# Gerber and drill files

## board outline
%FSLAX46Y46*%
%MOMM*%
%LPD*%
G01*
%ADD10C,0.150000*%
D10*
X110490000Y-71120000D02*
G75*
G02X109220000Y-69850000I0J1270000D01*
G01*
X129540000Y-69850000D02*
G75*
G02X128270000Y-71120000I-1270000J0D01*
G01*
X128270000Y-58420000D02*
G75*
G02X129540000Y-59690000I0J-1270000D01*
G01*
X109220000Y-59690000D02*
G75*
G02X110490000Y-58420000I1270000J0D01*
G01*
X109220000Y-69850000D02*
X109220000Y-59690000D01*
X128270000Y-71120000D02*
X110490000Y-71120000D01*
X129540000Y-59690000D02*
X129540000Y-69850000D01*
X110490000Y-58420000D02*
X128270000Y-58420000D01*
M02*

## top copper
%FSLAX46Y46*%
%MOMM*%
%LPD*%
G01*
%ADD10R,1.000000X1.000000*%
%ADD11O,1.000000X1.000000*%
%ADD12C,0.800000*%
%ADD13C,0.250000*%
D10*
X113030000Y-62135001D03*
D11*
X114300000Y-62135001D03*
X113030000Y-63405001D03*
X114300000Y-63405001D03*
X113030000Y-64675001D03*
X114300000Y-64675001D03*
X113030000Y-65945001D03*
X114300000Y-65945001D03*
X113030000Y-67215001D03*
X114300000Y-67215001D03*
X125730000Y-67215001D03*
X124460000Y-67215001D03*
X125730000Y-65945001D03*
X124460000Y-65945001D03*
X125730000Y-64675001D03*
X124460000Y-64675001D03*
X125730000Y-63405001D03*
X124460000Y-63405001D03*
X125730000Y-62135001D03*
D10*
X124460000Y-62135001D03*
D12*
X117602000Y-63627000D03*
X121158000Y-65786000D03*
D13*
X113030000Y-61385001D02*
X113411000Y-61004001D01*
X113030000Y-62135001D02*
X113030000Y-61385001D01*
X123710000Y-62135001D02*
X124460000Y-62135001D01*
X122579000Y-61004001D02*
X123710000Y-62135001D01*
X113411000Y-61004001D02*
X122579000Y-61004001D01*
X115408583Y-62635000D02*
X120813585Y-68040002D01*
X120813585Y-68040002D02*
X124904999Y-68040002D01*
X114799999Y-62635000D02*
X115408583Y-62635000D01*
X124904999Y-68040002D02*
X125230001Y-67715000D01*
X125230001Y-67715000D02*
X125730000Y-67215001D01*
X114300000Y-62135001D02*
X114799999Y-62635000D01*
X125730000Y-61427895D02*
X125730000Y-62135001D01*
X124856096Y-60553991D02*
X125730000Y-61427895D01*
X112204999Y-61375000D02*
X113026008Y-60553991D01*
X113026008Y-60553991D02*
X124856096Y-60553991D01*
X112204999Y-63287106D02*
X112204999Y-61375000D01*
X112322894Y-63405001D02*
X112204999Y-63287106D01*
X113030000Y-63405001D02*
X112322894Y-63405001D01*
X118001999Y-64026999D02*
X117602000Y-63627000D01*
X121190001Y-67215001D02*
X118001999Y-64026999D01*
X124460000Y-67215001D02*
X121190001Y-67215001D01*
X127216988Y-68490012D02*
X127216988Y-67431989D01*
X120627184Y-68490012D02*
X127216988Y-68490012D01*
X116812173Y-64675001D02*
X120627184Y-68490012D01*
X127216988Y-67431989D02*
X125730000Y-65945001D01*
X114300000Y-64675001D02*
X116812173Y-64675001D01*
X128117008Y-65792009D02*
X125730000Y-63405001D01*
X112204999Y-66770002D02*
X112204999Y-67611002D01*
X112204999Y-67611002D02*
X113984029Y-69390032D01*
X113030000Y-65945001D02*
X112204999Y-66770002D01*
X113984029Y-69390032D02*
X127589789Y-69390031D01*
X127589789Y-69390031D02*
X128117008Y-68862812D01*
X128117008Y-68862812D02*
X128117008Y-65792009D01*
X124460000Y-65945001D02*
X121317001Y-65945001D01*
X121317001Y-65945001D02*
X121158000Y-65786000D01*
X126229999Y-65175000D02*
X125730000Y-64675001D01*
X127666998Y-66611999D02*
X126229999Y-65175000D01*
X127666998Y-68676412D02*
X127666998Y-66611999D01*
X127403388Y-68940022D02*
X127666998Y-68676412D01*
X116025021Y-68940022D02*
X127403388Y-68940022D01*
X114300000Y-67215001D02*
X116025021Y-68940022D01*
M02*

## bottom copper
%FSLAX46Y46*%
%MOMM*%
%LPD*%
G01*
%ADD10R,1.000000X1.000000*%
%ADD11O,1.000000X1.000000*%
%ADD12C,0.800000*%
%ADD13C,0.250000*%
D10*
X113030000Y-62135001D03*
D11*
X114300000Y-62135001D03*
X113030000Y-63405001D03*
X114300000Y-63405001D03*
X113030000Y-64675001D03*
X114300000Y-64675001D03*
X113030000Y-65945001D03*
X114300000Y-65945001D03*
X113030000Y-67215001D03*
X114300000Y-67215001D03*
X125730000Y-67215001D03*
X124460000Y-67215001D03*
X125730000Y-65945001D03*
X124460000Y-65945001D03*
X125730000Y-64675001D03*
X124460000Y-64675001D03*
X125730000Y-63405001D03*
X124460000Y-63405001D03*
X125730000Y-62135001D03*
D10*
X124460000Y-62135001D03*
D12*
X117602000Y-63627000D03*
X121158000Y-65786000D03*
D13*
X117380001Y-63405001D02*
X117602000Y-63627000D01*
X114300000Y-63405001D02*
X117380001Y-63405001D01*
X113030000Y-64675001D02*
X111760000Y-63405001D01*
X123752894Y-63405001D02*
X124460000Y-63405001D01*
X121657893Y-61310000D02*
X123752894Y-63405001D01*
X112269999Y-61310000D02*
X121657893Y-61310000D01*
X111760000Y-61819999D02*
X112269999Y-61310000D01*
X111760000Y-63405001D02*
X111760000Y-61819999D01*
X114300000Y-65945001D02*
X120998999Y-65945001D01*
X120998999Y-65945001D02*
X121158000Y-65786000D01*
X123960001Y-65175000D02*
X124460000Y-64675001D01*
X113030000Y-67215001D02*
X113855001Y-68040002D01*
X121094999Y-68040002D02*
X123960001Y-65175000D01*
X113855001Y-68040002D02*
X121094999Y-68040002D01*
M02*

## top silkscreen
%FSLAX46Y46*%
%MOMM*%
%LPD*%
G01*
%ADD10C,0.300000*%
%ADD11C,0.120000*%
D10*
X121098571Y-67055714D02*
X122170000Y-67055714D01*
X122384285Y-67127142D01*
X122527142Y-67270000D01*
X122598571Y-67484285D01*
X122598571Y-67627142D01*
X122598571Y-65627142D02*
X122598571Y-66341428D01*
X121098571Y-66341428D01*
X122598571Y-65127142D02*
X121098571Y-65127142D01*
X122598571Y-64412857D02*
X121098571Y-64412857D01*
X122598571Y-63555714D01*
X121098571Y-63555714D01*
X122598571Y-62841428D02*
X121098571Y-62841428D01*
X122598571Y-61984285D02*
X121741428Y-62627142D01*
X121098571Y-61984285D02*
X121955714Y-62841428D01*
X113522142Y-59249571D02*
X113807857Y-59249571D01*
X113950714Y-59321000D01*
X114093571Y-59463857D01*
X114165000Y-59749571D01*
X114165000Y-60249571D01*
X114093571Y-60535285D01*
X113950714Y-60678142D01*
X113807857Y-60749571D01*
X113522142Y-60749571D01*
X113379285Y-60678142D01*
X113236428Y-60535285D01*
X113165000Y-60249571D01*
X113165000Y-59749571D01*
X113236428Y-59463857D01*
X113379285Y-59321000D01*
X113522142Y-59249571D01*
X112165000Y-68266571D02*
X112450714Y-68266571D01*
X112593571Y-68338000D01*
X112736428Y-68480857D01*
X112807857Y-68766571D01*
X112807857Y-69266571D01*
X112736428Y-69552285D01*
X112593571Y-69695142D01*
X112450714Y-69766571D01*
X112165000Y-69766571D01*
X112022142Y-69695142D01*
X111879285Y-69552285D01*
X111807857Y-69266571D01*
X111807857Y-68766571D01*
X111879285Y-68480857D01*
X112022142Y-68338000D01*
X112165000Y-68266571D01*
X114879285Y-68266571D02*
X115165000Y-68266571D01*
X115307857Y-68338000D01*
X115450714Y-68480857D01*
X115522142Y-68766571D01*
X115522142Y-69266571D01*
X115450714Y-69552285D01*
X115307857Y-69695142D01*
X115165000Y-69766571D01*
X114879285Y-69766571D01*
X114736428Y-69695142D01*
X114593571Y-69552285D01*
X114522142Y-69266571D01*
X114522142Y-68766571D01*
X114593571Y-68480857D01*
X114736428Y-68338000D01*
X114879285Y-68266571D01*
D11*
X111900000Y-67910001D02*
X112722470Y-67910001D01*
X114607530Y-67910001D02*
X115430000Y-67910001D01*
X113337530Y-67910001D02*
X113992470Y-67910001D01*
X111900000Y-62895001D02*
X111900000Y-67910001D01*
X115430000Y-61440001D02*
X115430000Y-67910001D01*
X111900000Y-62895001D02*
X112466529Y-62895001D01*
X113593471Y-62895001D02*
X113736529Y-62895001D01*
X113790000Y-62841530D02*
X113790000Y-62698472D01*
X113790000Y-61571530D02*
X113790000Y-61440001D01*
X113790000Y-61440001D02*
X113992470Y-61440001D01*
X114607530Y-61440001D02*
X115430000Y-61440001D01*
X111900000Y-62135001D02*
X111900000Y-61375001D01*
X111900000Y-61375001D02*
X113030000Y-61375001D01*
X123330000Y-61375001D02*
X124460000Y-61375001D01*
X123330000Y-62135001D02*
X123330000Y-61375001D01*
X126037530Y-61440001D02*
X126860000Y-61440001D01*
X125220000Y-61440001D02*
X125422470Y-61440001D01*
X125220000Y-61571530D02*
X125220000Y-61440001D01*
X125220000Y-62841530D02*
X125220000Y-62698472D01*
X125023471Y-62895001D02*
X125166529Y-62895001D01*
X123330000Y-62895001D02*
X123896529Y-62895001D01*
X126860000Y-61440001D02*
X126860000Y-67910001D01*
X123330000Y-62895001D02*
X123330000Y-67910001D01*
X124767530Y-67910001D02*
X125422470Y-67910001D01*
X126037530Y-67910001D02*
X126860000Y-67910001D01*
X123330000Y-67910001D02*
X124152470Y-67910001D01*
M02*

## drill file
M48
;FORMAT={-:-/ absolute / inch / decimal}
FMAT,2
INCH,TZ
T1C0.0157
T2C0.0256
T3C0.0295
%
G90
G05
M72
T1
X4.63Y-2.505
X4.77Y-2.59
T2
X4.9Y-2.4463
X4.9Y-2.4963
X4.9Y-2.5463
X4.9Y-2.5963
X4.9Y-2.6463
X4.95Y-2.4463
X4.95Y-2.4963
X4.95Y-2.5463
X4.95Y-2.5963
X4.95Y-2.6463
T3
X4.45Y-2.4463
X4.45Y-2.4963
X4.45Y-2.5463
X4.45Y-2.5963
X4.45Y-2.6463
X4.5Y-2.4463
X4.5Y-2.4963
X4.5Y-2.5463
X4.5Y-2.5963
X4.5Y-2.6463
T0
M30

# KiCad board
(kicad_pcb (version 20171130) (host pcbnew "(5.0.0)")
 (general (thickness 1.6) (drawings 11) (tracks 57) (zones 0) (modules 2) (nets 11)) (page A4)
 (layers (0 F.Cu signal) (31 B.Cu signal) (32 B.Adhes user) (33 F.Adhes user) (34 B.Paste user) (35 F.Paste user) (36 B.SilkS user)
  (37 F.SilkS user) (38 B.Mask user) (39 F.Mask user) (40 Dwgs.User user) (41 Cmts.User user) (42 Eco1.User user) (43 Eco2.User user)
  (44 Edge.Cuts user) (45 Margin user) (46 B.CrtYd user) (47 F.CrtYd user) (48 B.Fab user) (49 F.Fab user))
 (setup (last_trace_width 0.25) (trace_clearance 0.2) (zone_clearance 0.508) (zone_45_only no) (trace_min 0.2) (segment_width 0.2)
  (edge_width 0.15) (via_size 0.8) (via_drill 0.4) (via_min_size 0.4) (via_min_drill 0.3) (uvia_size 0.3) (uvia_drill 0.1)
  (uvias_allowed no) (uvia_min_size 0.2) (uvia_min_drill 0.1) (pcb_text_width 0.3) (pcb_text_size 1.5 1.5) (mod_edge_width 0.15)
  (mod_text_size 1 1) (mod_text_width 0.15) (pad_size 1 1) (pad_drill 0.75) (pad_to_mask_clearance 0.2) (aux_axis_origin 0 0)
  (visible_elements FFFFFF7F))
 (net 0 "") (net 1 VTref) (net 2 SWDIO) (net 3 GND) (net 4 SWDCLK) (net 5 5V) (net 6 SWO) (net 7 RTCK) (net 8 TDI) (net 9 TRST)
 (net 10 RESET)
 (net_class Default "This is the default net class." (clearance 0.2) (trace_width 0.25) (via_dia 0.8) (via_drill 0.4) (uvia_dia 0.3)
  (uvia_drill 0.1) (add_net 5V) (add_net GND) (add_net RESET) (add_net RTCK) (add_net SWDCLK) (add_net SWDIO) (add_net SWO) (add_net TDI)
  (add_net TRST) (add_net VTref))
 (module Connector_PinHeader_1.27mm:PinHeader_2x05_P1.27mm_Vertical (layer F.Cu) (at 113.03 62.135001)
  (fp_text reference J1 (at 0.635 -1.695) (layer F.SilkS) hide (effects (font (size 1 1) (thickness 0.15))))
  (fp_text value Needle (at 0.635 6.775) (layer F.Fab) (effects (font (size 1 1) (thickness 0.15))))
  (fp_line (start -1.13 5.775) (end -0.30753 5.775) (layer F.SilkS) (width 0.12))
  (fp_line (start 1.57753 5.775) (end 2.4 5.775) (layer F.SilkS) (width 0.12))
  (fp_line (start 0.30753 5.775) (end 0.96247 5.775) (layer F.SilkS) (width 0.12))
  (fp_line (start -1.13 0.76) (end -1.13 5.775) (layer F.SilkS) (width 0.12))
  (fp_line (start 2.4 -0.695) (end 2.4 5.775) (layer F.SilkS) (width 0.12))
  (fp_line (start -1.13 0.76) (end -0.563471 0.76) (layer F.SilkS) (width 0.12))
  (fp_line (start 0.563471 0.76) (end 0.706529 0.76) (layer F.SilkS) (width 0.12))
  (fp_line (start 0.76 0.706529) (end 0.76 0.563471) (layer F.SilkS) (width 0.12))
  (fp_line (start 0.76 -0.563471) (end 0.76 -0.695) (layer F.SilkS) (width 0.12))
  (fp_line (start 0.76 -0.695) (end 0.96247 -0.695) (layer F.SilkS) (width 0.12))
  (fp_line (start 1.57753 -0.695) (end 2.4 -0.695) (layer F.SilkS) (width 0.12))
  (fp_line (start -1.13 0) (end -1.13 -0.76) (layer F.SilkS) (width 0.12))
  (fp_line (start -1.13 -0.76) (end 0 -0.76) (layer F.SilkS) (width 0.12))
  (pad 1 thru_hole rect (at 0 0) (size 1 1) (drill 0.75) (layers *.Cu *.Mask) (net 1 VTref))
  (pad 2 thru_hole oval (at 1.27 0) (size 1 1) (drill 0.75) (layers *.Cu *.Mask) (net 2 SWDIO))
  (pad 3 thru_hole oval (at 0 1.27) (size 1 1) (drill 0.75) (layers *.Cu *.Mask) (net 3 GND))
  (pad 4 thru_hole oval (at 1.27 1.27) (size 1 1) (drill 0.75) (layers *.Cu *.Mask) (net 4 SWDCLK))
  (pad 5 thru_hole oval (at 0 2.54) (size 1 1) (drill 0.75) (layers *.Cu *.Mask) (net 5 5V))
  (pad 6 thru_hole oval (at 1.27 2.54) (size 1 1) (drill 0.75) (layers *.Cu *.Mask) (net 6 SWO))
  (pad 7 thru_hole oval (at 0 3.81) (size 1 1) (drill 0.75) (layers *.Cu *.Mask) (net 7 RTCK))
  (pad 8 thru_hole oval (at 1.27 3.81) (size 1 1) (drill 0.75) (layers *.Cu *.Mask) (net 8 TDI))
  (pad 9 thru_hole oval (at 0 5.08) (size 1 1) (drill 0.75) (layers *.Cu *.Mask) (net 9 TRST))
  (pad 10 thru_hole oval (at 1.27 5.08) (size 1 1) (drill 0.75) (layers *.Cu *.Mask) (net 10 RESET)))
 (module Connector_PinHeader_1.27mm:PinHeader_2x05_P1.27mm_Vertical (layer F.Cu) (at 124.46 62.135001)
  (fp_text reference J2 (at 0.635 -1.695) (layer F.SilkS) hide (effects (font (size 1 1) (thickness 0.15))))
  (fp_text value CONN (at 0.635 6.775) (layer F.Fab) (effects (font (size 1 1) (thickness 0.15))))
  (fp_line (start -1.13 -0.76) (end 0 -0.76) (layer F.SilkS) (width 0.12))
  (fp_line (start -1.13 0) (end -1.13 -0.76) (layer F.SilkS) (width 0.12))
  (fp_line (start 1.57753 -0.695) (end 2.4 -0.695) (layer F.SilkS) (width 0.12))
  (fp_line (start 0.76 -0.695) (end 0.96247 -0.695) (layer F.SilkS) (width 0.12))
  (fp_line (start 0.76 -0.563471) (end 0.76 -0.695) (layer F.SilkS) (width 0.12))
  (fp_line (start 0.76 0.706529) (end 0.76 0.563471) (layer F.SilkS) (width 0.12))
  (fp_line (start 0.563471 0.76) (end 0.706529 0.76) (layer F.SilkS) (width 0.12))
  (fp_line (start -1.13 0.76) (end -0.563471 0.76) (layer F.SilkS) (width 0.12))
  (fp_line (start 2.4 -0.695) (end 2.4 5.775) (layer F.SilkS) (width 0.12))
  (fp_line (start -1.13 0.76) (end -1.13 5.775) (layer F.SilkS) (width 0.12))
  (fp_line (start 0.30753 5.775) (end 0.96247 5.775) (layer F.SilkS) (width 0.12))
  (fp_line (start 1.57753 5.775) (end 2.4 5.775) (layer F.SilkS) (width 0.12))
  (fp_line (start -1.13 5.775) (end -0.30753 5.775) (layer F.SilkS) (width 0.12))
  (pad 10 thru_hole oval (at 1.27 5.08) (size 1 1) (drill 0.65) (layers *.Cu *.Mask) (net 2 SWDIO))
  (pad 9 thru_hole oval (at 0 5.08) (size 1 1) (drill 0.65) (layers *.Cu *.Mask) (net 4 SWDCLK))
  (pad 8 thru_hole oval (at 1.27 3.81) (size 1 1) (drill 0.65) (layers *.Cu *.Mask) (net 6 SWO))
  (pad 7 thru_hole oval (at 0 3.81) (size 1 1) (drill 0.65) (layers *.Cu *.Mask) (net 8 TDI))
  (pad 6 thru_hole oval (at 1.27 2.54) (size 1 1) (drill 0.65) (layers *.Cu *.Mask) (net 10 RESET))
  (pad 5 thru_hole oval (at 0 2.54) (size 1 1) (drill 0.65) (layers *.Cu *.Mask) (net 9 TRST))
  (pad 4 thru_hole oval (at 1.27 1.27) (size 1 1) (drill 0.65) (layers *.Cu *.Mask) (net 7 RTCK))
  (pad 3 thru_hole oval (at 0 1.27) (size 1 1) (drill 0.65) (layers *.Cu *.Mask) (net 5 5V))
  (pad 2 thru_hole oval (at 1.27 0) (size 1 1) (drill 0.65) (layers *.Cu *.Mask) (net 3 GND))
  (pad 1 thru_hole rect (at 0 0) (size 1 1) (drill 0.65) (layers *.Cu *.Mask) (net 1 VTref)))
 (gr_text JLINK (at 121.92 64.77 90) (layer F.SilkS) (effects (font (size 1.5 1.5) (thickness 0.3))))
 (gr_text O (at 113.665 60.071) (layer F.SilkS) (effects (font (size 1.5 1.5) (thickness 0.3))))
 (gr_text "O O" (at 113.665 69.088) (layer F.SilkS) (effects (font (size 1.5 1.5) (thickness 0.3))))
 (gr_arc (start 110.49 69.85) (end 109.22 69.85) (angle -90) (layer Edge.Cuts) (width 0.15))
 (gr_arc (start 128.27 69.85) (end 128.27 71.12) (angle -90) (layer Edge.Cuts) (width 0.15))
 (gr_arc (start 128.27 59.69) (end 129.54 59.69) (angle -90) (layer Edge.Cuts) (width 0.15))
 (gr_arc (start 110.49 59.69) (end 110.49 58.42) (angle -90) (layer Edge.Cuts) (width 0.15))
 (gr_line (start 109.22 69.85) (end 109.22 59.69) (layer Edge.Cuts) (width 0.15))
 (gr_line (start 128.27 71.12) (end 110.49 71.12) (layer Edge.Cuts) (width 0.15))
 (gr_line (start 129.54 59.69) (end 129.54 69.85) (layer Edge.Cuts) (width 0.15))
 (gr_line (start 110.49 58.42) (end 128.27 58.42) (layer Edge.Cuts) (width 0.15))
 (segment (start 113.03 61.385001) (end 113.411 61.004001) (width 0.25) (layer F.Cu) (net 1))
 (segment (start 113.03 62.135001) (end 113.03 61.385001) (width 0.25) (layer F.Cu) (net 1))
 (segment (start 123.71 62.135001) (end 124.46 62.135001) (width 0.25) (layer F.Cu) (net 1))
 (segment (start 122.579 61.004001) (end 123.71 62.135001) (width 0.25) (layer F.Cu) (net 1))
 (segment (start 113.411 61.004001) (end 122.579 61.004001) (width 0.25) (layer F.Cu) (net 1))
 (segment (start 115.408583 62.635) (end 120.813585 68.040002) (width 0.25) (layer F.Cu) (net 2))
 (segment (start 120.813585 68.040002) (end 124.904999 68.040002) (width 0.25) (layer F.Cu) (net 2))
 (segment (start 114.799999 62.635) (end 115.408583 62.635) (width 0.25) (layer F.Cu) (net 2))
 (segment (start 124.904999 68.040002) (end 125.230001 67.715) (width 0.25) (layer F.Cu) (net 2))
 (segment (start 125.230001 67.715) (end 125.73 67.215001) (width 0.25) (layer F.Cu) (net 2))
 (segment (start 114.3 62.135001) (end 114.799999 62.635) (width 0.25) (layer F.Cu) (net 2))
 (segment (start 125.73 61.427895) (end 125.73 62.135001) (width 0.25) (layer F.Cu) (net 3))
 (segment (start 124.856096 60.553991) (end 125.73 61.427895) (width 0.25) (layer F.Cu) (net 3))
 (segment (start 112.204999 61.375) (end 113.026008 60.553991) (width 0.25) (layer F.Cu) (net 3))
 (segment (start 113.026008 60.553991) (end 124.856096 60.553991) (width 0.25) (layer F.Cu) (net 3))
 (segment (start 112.204999 63.287106) (end 112.204999 61.375) (width 0.25) (layer F.Cu) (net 3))
 (segment (start 112.322894 63.405001) (end 112.204999 63.287106) (width 0.25) (layer F.Cu) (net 3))
 (segment (start 113.03 63.405001) (end 112.322894 63.405001) (width 0.25) (layer F.Cu) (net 3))
 (via (at 117.602 63.627) (size 0.8) (drill 0.4) (layers F.Cu B.Cu) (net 4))
 (segment (start 118.001999 64.026999) (end 117.602 63.627) (width 0.25) (layer F.Cu) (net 4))
 (segment (start 121.190001 67.215001) (end 118.001999 64.026999) (width 0.25) (layer F.Cu) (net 4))
 (segment (start 124.46 67.215001) (end 121.190001 67.215001) (width 0.25) (layer F.Cu) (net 4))
 (segment (start 117.380001 63.405001) (end 117.602 63.627) (width 0.25) (layer B.Cu) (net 4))
 (segment (start 114.3 63.405001) (end 117.380001 63.405001) (width 0.25) (layer B.Cu) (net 4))
 (segment (start 113.03 64.675001) (end 111.76 63.405001) (width 0.25) (layer B.Cu) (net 5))
 (segment (start 123.752894 63.405001) (end 124.46 63.405001) (width 0.25) (layer B.Cu) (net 5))
 (segment (start 121.657893 61.31) (end 123.752894 63.405001) (width 0.25) (layer B.Cu) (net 5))
 (segment (start 112.269999 61.31) (end 121.657893 61.31) (width 0.25) (layer B.Cu) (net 5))
 (segment (start 111.76 61.819999) (end 112.269999 61.31) (width 0.25) (layer B.Cu) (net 5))
 (segment (start 111.76 63.405001) (end 111.76 61.819999) (width 0.25) (layer B.Cu) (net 5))
 (segment (start 127.216988 68.490012) (end 127.216988 67.431989) (width 0.25) (layer F.Cu) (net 6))
 (segment (start 120.627184 68.490012) (end 127.216988 68.490012) (width 0.25) (layer F.Cu) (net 6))
 (segment (start 116.812173 64.675001) (end 120.627184 68.490012) (width 0.25) (layer F.Cu) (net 6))
 (segment (start 127.216988 67.431989) (end 125.73 65.945001) (width 0.25) (layer F.Cu) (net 6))
 (segment (start 114.3 64.675001) (end 116.812173 64.675001) (width 0.25) (layer F.Cu) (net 6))
 (segment (start 128.117008 65.792009) (end 125.73 63.405001) (width 0.25) (layer F.Cu) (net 7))
 (segment (start 112.204999 66.770002) (end 112.204999 67.611002) (width 0.25) (layer F.Cu) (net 7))
 (segment (start 112.204999 67.611002) (end 113.984029 69.390032) (width 0.25) (layer F.Cu) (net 7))
 (segment (start 113.03 65.945001) (end 112.204999 66.770002) (width 0.25) (layer F.Cu) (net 7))
 (segment (start 113.984029 69.390032) (end 127.589789 69.390031) (width 0.25) (layer F.Cu) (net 7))
 (segment (start 127.589789 69.390031) (end 128.117008 68.862812) (width 0.25) (layer F.Cu) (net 7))
 (segment (start 128.117008 68.862812) (end 128.117008 65.792009) (width 0.25) (layer F.Cu) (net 7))
 (segment (start 124.46 65.945001) (end 121.317001 65.945001) (width 0.25) (layer F.Cu) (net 8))
 (segment (start 114.3 65.945001) (end 120.998999 65.945001) (width 0.25) (layer B.Cu) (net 8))
 (via (at 121.158 65.786) (size 0.8) (drill 0.4) (layers F.Cu B.Cu) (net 8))
 (segment (start 121.317001 65.945001) (end 121.158 65.786) (width 0.25) (layer F.Cu) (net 8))
 (segment (start 120.998999 65.945001) (end 121.158 65.786) (width 0.25) (layer B.Cu) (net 8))
 (segment (start 123.960001 65.175) (end 124.46 64.675001) (width 0.25) (layer B.Cu) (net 9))
 (segment (start 113.03 67.215001) (end 113.855001 68.040002) (width 0.25) (layer B.Cu) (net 9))
 (segment (start 121.094999 68.040002) (end 123.960001 65.175) (width 0.25) (layer B.Cu) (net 9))
 (segment (start 113.855001 68.040002) (end 121.094999 68.040002) (width 0.25) (layer B.Cu) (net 9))
 (segment (start 126.229999 65.175) (end 125.73 64.675001) (width 0.25) (layer F.Cu) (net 10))
 (segment (start 127.666998 66.611999) (end 126.229999 65.175) (width 0.25) (layer F.Cu) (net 10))
 (segment (start 127.666998 68.676412) (end 127.666998 66.611999) (width 0.25) (layer F.Cu) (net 10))
 (segment (start 127.403388 68.940022) (end 127.666998 68.676412) (width 0.25) (layer F.Cu) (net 10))
 (segment (start 116.025021 68.940022) (end 127.403388 68.940022) (width 0.25) (layer F.Cu) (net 10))
 (segment (start 114.3 67.215001) (end 116.025021 68.940022) (width 0.25) (layer F.Cu) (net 10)))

